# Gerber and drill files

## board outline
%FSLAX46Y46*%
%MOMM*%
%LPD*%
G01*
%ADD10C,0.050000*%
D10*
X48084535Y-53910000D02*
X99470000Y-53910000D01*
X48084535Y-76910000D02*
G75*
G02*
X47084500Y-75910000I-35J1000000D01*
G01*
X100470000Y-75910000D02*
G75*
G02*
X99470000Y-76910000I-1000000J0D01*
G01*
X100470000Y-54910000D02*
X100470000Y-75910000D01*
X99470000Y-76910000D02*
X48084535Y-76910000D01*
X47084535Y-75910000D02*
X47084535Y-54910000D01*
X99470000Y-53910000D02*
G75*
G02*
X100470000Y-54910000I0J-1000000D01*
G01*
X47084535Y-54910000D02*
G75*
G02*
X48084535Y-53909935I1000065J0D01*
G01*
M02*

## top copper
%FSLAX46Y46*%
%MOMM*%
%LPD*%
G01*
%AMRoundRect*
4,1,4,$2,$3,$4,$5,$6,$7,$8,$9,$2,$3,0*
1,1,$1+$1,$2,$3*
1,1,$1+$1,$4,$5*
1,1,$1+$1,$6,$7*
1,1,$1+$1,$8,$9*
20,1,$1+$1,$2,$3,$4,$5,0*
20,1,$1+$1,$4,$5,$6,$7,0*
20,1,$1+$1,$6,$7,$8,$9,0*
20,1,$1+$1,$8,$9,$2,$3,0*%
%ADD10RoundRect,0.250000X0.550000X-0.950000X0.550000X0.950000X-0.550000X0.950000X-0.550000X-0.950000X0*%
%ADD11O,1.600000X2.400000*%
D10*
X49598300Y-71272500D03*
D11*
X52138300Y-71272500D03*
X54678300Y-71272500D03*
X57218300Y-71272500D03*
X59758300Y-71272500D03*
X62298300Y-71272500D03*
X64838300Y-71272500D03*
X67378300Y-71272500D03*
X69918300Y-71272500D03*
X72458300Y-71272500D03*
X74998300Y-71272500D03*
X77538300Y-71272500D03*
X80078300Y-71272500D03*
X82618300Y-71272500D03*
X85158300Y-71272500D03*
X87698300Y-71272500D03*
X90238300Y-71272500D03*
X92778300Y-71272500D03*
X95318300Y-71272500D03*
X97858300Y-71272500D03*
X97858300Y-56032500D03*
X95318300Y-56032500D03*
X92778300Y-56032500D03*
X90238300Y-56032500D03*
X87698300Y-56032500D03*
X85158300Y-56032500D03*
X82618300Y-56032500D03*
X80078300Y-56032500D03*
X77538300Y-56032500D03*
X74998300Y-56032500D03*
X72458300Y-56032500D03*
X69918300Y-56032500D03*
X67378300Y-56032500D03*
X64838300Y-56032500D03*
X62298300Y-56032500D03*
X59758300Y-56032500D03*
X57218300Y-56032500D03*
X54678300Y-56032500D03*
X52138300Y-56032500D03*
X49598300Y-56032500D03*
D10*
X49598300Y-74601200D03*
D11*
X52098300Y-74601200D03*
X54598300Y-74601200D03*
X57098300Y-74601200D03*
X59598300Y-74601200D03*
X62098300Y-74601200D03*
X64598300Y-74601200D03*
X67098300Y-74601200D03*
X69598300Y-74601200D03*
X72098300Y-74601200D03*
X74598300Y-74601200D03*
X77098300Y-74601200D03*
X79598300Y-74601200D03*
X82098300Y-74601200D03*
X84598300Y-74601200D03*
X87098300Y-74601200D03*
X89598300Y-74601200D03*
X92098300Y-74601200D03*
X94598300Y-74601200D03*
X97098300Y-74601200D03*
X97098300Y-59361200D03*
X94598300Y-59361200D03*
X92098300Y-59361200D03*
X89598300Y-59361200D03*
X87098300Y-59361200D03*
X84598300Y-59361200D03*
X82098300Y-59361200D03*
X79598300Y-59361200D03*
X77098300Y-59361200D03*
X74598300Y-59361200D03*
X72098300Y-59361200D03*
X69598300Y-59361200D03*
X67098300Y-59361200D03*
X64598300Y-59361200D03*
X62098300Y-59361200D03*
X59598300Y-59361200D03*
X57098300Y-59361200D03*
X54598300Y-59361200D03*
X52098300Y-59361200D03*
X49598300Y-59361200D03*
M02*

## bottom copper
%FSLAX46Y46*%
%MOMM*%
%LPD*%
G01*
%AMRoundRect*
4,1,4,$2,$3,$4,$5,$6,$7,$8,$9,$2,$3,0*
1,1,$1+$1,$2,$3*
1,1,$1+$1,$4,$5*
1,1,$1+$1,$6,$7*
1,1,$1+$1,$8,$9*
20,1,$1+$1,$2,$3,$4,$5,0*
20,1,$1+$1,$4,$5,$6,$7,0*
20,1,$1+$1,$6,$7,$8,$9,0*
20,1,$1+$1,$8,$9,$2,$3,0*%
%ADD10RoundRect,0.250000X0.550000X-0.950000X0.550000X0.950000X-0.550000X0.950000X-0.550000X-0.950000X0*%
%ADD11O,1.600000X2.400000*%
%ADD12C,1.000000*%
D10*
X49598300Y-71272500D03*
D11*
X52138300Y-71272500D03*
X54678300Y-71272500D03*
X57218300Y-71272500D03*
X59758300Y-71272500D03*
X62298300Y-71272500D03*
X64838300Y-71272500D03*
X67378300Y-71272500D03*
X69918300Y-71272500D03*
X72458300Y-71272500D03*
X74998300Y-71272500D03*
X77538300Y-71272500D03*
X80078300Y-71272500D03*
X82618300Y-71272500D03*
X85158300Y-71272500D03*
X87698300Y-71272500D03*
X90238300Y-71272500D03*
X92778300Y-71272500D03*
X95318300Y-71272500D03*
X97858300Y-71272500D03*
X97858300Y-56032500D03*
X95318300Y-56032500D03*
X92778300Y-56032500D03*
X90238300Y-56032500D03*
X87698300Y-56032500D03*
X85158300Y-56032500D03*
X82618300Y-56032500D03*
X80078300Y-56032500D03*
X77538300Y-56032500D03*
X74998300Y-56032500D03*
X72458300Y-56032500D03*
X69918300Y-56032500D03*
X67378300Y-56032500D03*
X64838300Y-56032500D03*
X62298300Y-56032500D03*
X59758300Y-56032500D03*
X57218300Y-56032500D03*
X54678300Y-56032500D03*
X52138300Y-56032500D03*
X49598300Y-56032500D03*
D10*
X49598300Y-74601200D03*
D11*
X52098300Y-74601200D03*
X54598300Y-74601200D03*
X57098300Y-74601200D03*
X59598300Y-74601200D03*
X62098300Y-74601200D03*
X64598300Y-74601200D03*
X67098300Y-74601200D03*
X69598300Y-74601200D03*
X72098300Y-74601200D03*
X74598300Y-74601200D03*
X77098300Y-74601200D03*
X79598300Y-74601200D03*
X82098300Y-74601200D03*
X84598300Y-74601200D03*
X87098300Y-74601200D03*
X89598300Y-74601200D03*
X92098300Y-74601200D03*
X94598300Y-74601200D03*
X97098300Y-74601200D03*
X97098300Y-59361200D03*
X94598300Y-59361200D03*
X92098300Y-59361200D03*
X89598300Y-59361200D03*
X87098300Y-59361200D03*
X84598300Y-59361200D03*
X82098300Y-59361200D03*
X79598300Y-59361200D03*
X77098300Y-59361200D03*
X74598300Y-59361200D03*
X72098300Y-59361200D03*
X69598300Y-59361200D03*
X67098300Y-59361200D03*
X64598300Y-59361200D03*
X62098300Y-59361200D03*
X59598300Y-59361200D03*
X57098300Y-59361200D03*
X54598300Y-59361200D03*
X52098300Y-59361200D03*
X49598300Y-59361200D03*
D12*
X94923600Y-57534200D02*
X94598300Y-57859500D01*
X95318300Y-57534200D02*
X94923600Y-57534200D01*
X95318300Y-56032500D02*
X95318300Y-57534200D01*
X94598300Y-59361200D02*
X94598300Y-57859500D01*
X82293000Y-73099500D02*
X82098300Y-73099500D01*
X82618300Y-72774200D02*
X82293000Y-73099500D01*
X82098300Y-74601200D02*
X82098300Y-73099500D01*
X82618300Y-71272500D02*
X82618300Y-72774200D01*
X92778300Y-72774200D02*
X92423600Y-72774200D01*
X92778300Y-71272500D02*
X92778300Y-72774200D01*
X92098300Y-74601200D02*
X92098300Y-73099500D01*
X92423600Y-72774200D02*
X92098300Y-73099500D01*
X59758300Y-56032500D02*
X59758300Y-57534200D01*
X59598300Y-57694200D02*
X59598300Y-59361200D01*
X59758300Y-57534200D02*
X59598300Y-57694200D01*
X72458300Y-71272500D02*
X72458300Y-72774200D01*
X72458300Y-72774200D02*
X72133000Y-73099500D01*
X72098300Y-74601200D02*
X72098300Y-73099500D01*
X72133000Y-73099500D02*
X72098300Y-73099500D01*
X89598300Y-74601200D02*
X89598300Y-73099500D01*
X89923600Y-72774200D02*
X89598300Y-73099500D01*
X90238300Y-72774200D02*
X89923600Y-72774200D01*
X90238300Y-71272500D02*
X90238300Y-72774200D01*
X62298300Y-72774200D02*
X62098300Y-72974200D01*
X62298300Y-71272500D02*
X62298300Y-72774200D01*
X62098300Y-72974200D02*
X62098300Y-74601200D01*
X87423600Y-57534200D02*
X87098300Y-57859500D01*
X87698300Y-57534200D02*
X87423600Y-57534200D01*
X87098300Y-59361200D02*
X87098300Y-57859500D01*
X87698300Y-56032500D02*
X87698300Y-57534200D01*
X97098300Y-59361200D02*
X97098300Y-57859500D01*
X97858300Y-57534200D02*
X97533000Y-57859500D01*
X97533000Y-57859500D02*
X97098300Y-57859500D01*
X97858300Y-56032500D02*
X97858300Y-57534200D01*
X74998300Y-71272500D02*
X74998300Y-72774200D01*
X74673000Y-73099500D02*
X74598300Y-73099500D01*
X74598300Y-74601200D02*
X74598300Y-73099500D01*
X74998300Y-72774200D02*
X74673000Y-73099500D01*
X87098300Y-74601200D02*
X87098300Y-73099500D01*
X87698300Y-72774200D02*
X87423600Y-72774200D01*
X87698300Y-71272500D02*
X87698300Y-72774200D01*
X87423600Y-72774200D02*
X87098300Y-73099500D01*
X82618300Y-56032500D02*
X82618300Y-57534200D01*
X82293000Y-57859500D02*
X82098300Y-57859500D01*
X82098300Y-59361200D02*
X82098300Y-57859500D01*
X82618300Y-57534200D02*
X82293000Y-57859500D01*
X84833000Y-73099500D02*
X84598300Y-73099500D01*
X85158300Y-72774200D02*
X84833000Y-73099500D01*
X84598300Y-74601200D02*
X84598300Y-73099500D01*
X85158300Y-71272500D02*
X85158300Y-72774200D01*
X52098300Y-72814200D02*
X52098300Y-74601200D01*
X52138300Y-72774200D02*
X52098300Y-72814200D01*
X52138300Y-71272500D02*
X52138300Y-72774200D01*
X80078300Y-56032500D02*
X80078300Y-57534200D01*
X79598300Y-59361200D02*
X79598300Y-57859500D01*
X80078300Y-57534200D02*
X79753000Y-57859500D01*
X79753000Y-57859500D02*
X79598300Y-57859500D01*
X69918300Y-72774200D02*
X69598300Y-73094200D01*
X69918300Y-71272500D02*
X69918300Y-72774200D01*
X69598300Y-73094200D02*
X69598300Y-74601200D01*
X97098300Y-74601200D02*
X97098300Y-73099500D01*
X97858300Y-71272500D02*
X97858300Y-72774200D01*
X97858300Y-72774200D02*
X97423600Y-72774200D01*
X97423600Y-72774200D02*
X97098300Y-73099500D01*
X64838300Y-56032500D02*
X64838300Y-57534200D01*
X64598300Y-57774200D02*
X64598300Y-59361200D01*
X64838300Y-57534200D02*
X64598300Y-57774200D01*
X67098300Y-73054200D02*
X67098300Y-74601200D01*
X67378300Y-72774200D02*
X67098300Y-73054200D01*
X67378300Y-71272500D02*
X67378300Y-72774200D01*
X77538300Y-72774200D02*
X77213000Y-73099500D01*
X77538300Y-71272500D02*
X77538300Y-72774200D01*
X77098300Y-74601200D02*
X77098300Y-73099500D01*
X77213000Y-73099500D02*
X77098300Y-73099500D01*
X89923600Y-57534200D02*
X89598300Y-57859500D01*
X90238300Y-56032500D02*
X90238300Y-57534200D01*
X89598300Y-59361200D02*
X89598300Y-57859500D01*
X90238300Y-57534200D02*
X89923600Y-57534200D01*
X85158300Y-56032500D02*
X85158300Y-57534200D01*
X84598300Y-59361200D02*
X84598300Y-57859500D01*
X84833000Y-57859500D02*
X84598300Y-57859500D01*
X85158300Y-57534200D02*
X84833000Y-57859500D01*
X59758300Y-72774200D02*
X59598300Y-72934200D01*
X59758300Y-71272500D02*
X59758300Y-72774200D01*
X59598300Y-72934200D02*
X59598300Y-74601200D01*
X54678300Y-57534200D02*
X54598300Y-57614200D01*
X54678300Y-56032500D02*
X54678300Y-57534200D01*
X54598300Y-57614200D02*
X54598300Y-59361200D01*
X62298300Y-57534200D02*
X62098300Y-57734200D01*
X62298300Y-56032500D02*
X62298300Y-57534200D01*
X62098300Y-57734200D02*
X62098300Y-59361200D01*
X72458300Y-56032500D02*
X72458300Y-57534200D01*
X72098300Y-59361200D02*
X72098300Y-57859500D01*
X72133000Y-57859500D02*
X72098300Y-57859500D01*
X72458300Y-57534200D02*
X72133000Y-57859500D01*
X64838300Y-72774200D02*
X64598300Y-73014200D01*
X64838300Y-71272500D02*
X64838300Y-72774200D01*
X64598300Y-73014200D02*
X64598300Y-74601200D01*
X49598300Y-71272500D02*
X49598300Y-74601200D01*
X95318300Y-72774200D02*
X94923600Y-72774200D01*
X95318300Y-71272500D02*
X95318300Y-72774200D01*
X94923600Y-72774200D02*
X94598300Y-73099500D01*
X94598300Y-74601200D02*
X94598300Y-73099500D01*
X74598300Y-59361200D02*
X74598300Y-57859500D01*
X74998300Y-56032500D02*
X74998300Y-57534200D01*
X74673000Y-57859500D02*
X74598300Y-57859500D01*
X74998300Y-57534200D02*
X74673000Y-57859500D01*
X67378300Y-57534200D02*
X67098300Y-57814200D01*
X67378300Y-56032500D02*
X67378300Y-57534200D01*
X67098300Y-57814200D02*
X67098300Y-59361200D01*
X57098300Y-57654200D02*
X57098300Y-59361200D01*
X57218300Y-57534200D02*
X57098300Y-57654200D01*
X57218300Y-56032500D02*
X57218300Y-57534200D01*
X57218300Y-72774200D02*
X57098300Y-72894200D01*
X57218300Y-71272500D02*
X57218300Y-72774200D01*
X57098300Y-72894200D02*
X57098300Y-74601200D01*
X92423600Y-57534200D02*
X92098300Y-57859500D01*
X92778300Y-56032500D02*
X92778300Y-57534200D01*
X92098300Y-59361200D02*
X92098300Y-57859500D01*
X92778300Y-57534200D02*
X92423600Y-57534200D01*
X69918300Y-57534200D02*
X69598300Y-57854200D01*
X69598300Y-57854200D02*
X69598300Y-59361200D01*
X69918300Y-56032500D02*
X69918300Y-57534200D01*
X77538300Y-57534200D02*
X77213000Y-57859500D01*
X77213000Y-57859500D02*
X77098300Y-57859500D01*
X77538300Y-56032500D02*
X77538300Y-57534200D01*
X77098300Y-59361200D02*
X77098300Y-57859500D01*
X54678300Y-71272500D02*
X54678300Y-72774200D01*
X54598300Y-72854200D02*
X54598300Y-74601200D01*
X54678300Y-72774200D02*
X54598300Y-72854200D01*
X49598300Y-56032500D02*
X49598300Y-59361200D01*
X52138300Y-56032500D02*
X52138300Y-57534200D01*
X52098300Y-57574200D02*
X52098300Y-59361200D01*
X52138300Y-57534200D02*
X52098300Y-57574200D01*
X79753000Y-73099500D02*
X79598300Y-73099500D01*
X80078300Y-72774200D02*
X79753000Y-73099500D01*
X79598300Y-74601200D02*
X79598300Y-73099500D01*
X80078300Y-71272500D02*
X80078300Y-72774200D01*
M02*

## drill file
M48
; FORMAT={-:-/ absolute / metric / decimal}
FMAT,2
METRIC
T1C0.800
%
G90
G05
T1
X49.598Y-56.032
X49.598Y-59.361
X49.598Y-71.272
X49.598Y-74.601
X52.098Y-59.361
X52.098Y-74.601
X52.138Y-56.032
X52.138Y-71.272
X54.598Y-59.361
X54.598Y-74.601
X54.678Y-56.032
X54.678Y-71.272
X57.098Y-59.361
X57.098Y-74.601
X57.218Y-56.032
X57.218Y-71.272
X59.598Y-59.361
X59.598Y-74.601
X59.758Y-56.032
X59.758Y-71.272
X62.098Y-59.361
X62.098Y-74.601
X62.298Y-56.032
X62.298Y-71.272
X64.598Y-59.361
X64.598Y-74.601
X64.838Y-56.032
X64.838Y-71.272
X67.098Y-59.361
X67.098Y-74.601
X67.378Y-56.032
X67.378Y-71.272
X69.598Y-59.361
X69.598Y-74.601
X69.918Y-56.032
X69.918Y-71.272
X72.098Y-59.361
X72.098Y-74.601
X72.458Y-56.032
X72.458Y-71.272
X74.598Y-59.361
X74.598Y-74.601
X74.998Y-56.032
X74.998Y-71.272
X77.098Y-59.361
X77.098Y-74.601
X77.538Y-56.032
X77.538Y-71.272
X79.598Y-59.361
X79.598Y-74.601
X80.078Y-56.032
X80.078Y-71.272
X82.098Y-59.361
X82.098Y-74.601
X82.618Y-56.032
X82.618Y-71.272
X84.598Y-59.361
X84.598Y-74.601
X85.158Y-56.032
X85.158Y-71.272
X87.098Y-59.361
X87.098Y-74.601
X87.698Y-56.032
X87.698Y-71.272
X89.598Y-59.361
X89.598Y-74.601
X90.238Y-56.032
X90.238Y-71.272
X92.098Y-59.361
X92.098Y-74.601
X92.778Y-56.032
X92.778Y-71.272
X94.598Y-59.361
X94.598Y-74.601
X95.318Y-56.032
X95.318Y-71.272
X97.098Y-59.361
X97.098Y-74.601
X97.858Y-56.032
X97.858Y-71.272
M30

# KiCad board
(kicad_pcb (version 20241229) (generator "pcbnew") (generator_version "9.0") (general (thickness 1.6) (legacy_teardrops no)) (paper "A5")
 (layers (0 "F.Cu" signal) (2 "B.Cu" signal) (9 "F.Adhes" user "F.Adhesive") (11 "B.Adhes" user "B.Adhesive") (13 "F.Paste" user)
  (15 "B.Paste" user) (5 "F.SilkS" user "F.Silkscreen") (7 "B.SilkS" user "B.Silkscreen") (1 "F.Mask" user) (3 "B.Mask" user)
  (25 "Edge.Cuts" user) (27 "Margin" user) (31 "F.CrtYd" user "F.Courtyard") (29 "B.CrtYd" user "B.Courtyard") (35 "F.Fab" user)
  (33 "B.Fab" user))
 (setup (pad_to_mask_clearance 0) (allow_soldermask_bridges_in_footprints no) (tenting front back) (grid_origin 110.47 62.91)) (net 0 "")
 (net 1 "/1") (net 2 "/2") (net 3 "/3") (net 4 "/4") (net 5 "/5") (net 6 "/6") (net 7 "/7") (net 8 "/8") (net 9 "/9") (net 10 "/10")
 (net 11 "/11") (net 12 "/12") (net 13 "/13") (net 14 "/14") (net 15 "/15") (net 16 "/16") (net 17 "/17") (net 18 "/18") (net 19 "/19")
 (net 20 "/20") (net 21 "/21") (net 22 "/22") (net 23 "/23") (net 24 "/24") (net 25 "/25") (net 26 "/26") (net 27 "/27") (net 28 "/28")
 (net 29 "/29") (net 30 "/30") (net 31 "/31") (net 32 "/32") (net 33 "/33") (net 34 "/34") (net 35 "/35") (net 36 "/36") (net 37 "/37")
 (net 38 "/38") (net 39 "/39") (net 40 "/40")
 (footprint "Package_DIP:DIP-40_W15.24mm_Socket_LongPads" (layer "F.Cu") (at 49.5983 71.2725 90)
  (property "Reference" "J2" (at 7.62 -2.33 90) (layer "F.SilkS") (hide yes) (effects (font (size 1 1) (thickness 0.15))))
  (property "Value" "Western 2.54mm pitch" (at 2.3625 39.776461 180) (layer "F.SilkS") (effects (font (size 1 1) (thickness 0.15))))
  (pad "1" thru_hole roundrect (at 0 0 90) (size 2.4 1.6) (drill 0.8) (layers "*.Cu" "*.Mask") (remove_unused_layers no)
   (roundrect_rratio 0.15625) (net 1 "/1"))
  (pad "2" thru_hole oval (at 0 2.54 90) (size 2.4 1.6) (drill 0.8) (layers "*.Cu" "*.Mask") (remove_unused_layers no) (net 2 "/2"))
  (pad "3" thru_hole oval (at 0 5.08 90) (size 2.4 1.6) (drill 0.8) (layers "*.Cu" "*.Mask") (remove_unused_layers no) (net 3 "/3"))
  (pad "4" thru_hole oval (at 0 7.62 90) (size 2.4 1.6) (drill 0.8) (layers "*.Cu" "*.Mask") (remove_unused_layers no) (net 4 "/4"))
  (pad "5" thru_hole oval (at 0 10.16 90) (size 2.4 1.6) (drill 0.8) (layers "*.Cu" "*.Mask") (remove_unused_layers no) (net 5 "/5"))
  (pad "6" thru_hole oval (at 0 12.7 90) (size 2.4 1.6) (drill 0.8) (layers "*.Cu" "*.Mask") (remove_unused_layers no) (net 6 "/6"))
  (pad "7" thru_hole oval (at 0 15.24 90) (size 2.4 1.6) (drill 0.8) (layers "*.Cu" "*.Mask") (remove_unused_layers no) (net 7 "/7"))
  (pad "8" thru_hole oval (at 0 17.78 90) (size 2.4 1.6) (drill 0.8) (layers "*.Cu" "*.Mask") (remove_unused_layers no) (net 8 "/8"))
  (pad "9" thru_hole oval (at 0 20.32 90) (size 2.4 1.6) (drill 0.8) (layers "*.Cu" "*.Mask") (remove_unused_layers no) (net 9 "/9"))
  (pad "10" thru_hole oval (at 0 22.86 90) (size 2.4 1.6) (drill 0.8) (layers "*.Cu" "*.Mask") (remove_unused_layers no) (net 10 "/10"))
  (pad "11" thru_hole oval (at 0 25.4 90) (size 2.4 1.6) (drill 0.8) (layers "*.Cu" "*.Mask") (remove_unused_layers no) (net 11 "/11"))
  (pad "12" thru_hole oval (at 0 27.94 90) (size 2.4 1.6) (drill 0.8) (layers "*.Cu" "*.Mask") (remove_unused_layers no) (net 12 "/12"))
  (pad "13" thru_hole oval (at 0 30.48 90) (size 2.4 1.6) (drill 0.8) (layers "*.Cu" "*.Mask") (remove_unused_layers no) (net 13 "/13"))
  (pad "14" thru_hole oval (at 0 33.02 90) (size 2.4 1.6) (drill 0.8) (layers "*.Cu" "*.Mask") (remove_unused_layers no) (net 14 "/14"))
  (pad "15" thru_hole oval (at 0 35.56 90) (size 2.4 1.6) (drill 0.8) (layers "*.Cu" "*.Mask") (remove_unused_layers no) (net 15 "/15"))
  (pad "16" thru_hole oval (at 0 38.1 90) (size 2.4 1.6) (drill 0.8) (layers "*.Cu" "*.Mask") (remove_unused_layers no) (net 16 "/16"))
  (pad "17" thru_hole oval (at 0 40.64 90) (size 2.4 1.6) (drill 0.8) (layers "*.Cu" "*.Mask") (remove_unused_layers no) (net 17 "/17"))
  (pad "18" thru_hole oval (at 0 43.18 90) (size 2.4 1.6) (drill 0.8) (layers "*.Cu" "*.Mask") (remove_unused_layers no) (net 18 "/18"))
  (pad "19" thru_hole oval (at 0 45.72 90) (size 2.4 1.6) (drill 0.8) (layers "*.Cu" "*.Mask") (remove_unused_layers no) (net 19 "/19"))
  (pad "20" thru_hole oval (at 0 48.26 90) (size 2.4 1.6) (drill 0.8) (layers "*.Cu" "*.Mask") (remove_unused_layers no) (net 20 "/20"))
  (pad "21" thru_hole oval (at 15.24 48.26 90) (size 2.4 1.6) (drill 0.8) (layers "*.Cu" "*.Mask") (remove_unused_layers no) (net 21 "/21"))
  (pad "22" thru_hole oval (at 15.24 45.72 90) (size 2.4 1.6) (drill 0.8) (layers "*.Cu" "*.Mask") (remove_unused_layers no) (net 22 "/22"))
  (pad "23" thru_hole oval (at 15.24 43.18 90) (size 2.4 1.6) (drill 0.8) (layers "*.Cu" "*.Mask") (remove_unused_layers no) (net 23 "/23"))
  (pad "24" thru_hole oval (at 15.24 40.64 90) (size 2.4 1.6) (drill 0.8) (layers "*.Cu" "*.Mask") (remove_unused_layers no) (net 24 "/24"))
  (pad "25" thru_hole oval (at 15.24 38.1 90) (size 2.4 1.6) (drill 0.8) (layers "*.Cu" "*.Mask") (remove_unused_layers no) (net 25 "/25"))
  (pad "26" thru_hole oval (at 15.24 35.56 90) (size 2.4 1.6) (drill 0.8) (layers "*.Cu" "*.Mask") (remove_unused_layers no) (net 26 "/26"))
  (pad "27" thru_hole oval (at 15.24 33.02 90) (size 2.4 1.6) (drill 0.8) (layers "*.Cu" "*.Mask") (remove_unused_layers no) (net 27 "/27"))
  (pad "28" thru_hole oval (at 15.24 30.48 90) (size 2.4 1.6) (drill 0.8) (layers "*.Cu" "*.Mask") (remove_unused_layers no) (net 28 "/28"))
  (pad "29" thru_hole oval (at 15.24 27.94 90) (size 2.4 1.6) (drill 0.8) (layers "*.Cu" "*.Mask") (remove_unused_layers no) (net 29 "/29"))
  (pad "30" thru_hole oval (at 15.24 25.4 90) (size 2.4 1.6) (drill 0.8) (layers "*.Cu" "*.Mask") (remove_unused_layers no) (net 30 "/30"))
  (pad "31" thru_hole oval (at 15.24 22.86 90) (size 2.4 1.6) (drill 0.8) (layers "*.Cu" "*.Mask") (remove_unused_layers no) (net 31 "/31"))
  (pad "32" thru_hole oval (at 15.24 20.32 90) (size 2.4 1.6) (drill 0.8) (layers "*.Cu" "*.Mask") (remove_unused_layers no) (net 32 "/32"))
  (pad "33" thru_hole oval (at 15.24 17.78 90) (size 2.4 1.6) (drill 0.8) (layers "*.Cu" "*.Mask") (remove_unused_layers no) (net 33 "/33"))
  (pad "34" thru_hole oval (at 15.24 15.24 90) (size 2.4 1.6) (drill 0.8) (layers "*.Cu" "*.Mask") (remove_unused_layers no) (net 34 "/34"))
  (pad "35" thru_hole oval (at 15.24 12.7 90) (size 2.4 1.6) (drill 0.8) (layers "*.Cu" "*.Mask") (remove_unused_layers no) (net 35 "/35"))
  (pad "36" thru_hole oval (at 15.24 10.16 90) (size 2.4 1.6) (drill 0.8) (layers "*.Cu" "*.Mask") (remove_unused_layers no) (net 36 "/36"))
  (pad "37" thru_hole oval (at 15.24 7.62 90) (size 2.4 1.6) (drill 0.8) (layers "*.Cu" "*.Mask") (remove_unused_layers no) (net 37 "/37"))
  (pad "38" thru_hole oval (at 15.24 5.08 90) (size 2.4 1.6) (drill 0.8) (layers "*.Cu" "*.Mask") (remove_unused_layers no) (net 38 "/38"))
  (pad "39" thru_hole oval (at 15.24 2.54 90) (size 2.4 1.6) (drill 0.8) (layers "*.Cu" "*.Mask") (remove_unused_layers no) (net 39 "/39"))
  (pad "40" thru_hole oval (at 15.24 0 90) (size 2.4 1.6) (drill 0.8) (layers "*.Cu" "*.Mask") (remove_unused_layers no) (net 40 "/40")))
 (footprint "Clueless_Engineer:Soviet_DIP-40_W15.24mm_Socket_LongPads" (layer "F.Cu") (at 49.5983 74.6012 90)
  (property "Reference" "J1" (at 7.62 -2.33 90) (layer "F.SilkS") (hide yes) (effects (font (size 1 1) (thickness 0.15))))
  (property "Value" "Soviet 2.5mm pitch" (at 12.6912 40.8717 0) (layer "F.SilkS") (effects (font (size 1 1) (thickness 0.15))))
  (pad "1" thru_hole roundrect (at 0 0 90) (size 2.4 1.6) (drill 0.8) (layers "*.Cu" "*.Mask") (remove_unused_layers no)
   (roundrect_rratio 0.15625) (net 1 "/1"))
  (pad "2" thru_hole oval (at 0 2.5 90) (size 2.4 1.6) (drill 0.8) (layers "*.Cu" "*.Mask") (remove_unused_layers no) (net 2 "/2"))
  (pad "3" thru_hole oval (at 0 5 90) (size 2.4 1.6) (drill 0.8) (layers "*.Cu" "*.Mask") (remove_unused_layers no) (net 3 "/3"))
  (pad "4" thru_hole oval (at 0 7.5 90) (size 2.4 1.6) (drill 0.8) (layers "*.Cu" "*.Mask") (remove_unused_layers no) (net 4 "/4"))
  (pad "5" thru_hole oval (at 0 10 90) (size 2.4 1.6) (drill 0.8) (layers "*.Cu" "*.Mask") (remove_unused_layers no) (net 5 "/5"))
  (pad "6" thru_hole oval (at 0 12.5 90) (size 2.4 1.6) (drill 0.8) (layers "*.Cu" "*.Mask") (remove_unused_layers no) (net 6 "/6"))
  (pad "7" thru_hole oval (at 0 15 90) (size 2.4 1.6) (drill 0.8) (layers "*.Cu" "*.Mask") (remove_unused_layers no) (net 7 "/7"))
  (pad "8" thru_hole oval (at 0 17.5 90) (size 2.4 1.6) (drill 0.8) (layers "*.Cu" "*.Mask") (remove_unused_layers no) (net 8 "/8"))
  (pad "9" thru_hole oval (at 0 20 90) (size 2.4 1.6) (drill 0.8) (layers "*.Cu" "*.Mask") (remove_unused_layers no) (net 9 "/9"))
  (pad "10" thru_hole oval (at 0 22.5 90) (size 2.4 1.6) (drill 0.8) (layers "*.Cu" "*.Mask") (remove_unused_layers no) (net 10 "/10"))
  (pad "11" thru_hole oval (at 0 25 90) (size 2.4 1.6) (drill 0.8) (layers "*.Cu" "*.Mask") (remove_unused_layers no) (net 11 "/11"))
  (pad "12" thru_hole oval (at 0 27.5 90) (size 2.4 1.6) (drill 0.8) (layers "*.Cu" "*.Mask") (remove_unused_layers no) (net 12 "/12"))
  (pad "13" thru_hole oval (at 0 30 90) (size 2.4 1.6) (drill 0.8) (layers "*.Cu" "*.Mask") (remove_unused_layers no) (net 13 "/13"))
  (pad "14" thru_hole oval (at 0 32.5 90) (size 2.4 1.6) (drill 0.8) (layers "*.Cu" "*.Mask") (remove_unused_layers no) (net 14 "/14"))
  (pad "15" thru_hole oval (at 0 35 90) (size 2.4 1.6) (drill 0.8) (layers "*.Cu" "*.Mask") (remove_unused_layers no) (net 15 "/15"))
  (pad "16" thru_hole oval (at 0 37.5 90) (size 2.4 1.6) (drill 0.8) (layers "*.Cu" "*.Mask") (remove_unused_layers no) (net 16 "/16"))
  (pad "17" thru_hole oval (at 0 40 90) (size 2.4 1.6) (drill 0.8) (layers "*.Cu" "*.Mask") (remove_unused_layers no) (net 17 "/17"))
  (pad "18" thru_hole oval (at 0 42.5 90) (size 2.4 1.6) (drill 0.8) (layers "*.Cu" "*.Mask") (remove_unused_layers no) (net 18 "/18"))
  (pad "19" thru_hole oval (at 0 45 90) (size 2.4 1.6) (drill 0.8) (layers "*.Cu" "*.Mask") (remove_unused_layers no) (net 19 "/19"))
  (pad "20" thru_hole oval (at 0 47.5 90) (size 2.4 1.6) (drill 0.8) (layers "*.Cu" "*.Mask") (remove_unused_layers no) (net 20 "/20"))
  (pad "21" thru_hole oval (at 15.24 47.5 90) (size 2.4 1.6) (drill 0.8) (layers "*.Cu" "*.Mask") (remove_unused_layers no) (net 21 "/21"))
  (pad "22" thru_hole oval (at 15.24 45 90) (size 2.4 1.6) (drill 0.8) (layers "*.Cu" "*.Mask") (remove_unused_layers no) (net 22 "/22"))
  (pad "23" thru_hole oval (at 15.24 42.5 90) (size 2.4 1.6) (drill 0.8) (layers "*.Cu" "*.Mask") (remove_unused_layers no) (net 23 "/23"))
  (pad "24" thru_hole oval (at 15.24 40 90) (size 2.4 1.6) (drill 0.8) (layers "*.Cu" "*.Mask") (remove_unused_layers no) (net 24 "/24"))
  (pad "25" thru_hole oval (at 15.24 37.5 90) (size 2.4 1.6) (drill 0.8) (layers "*.Cu" "*.Mask") (remove_unused_layers no) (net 25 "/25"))
  (pad "26" thru_hole oval (at 15.24 35 90) (size 2.4 1.6) (drill 0.8) (layers "*.Cu" "*.Mask") (remove_unused_layers no) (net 26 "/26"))
  (pad "27" thru_hole oval (at 15.24 32.5 90) (size 2.4 1.6) (drill 0.8) (layers "*.Cu" "*.Mask") (remove_unused_layers no) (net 27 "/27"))
  (pad "28" thru_hole oval (at 15.24 30 90) (size 2.4 1.6) (drill 0.8) (layers "*.Cu" "*.Mask") (remove_unused_layers no) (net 28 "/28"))
  (pad "29" thru_hole oval (at 15.24 27.5 90) (size 2.4 1.6) (drill 0.8) (layers "*.Cu" "*.Mask") (remove_unused_layers no) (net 29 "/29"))
  (pad "30" thru_hole oval (at 15.24 25 90) (size 2.4 1.6) (drill 0.8) (layers "*.Cu" "*.Mask") (remove_unused_layers no) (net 30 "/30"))
  (pad "31" thru_hole oval (at 15.24 22.5 90) (size 2.4 1.6) (drill 0.8) (layers "*.Cu" "*.Mask") (remove_unused_layers no) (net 31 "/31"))
  (pad "32" thru_hole oval (at 15.24 20 90) (size 2.4 1.6) (drill 0.8) (layers "*.Cu" "*.Mask") (remove_unused_layers no) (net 32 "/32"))
  (pad "33" thru_hole oval (at 15.24 17.5 90) (size 2.4 1.6) (drill 0.8) (layers "*.Cu" "*.Mask") (remove_unused_layers no) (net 33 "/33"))
  (pad "34" thru_hole oval (at 15.24 15 90) (size 2.4 1.6) (drill 0.8) (layers "*.Cu" "*.Mask") (remove_unused_layers no) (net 34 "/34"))
  (pad "35" thru_hole oval (at 15.24 12.5 90) (size 2.4 1.6) (drill 0.8) (layers "*.Cu" "*.Mask") (remove_unused_layers no) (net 35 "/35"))
  (pad "36" thru_hole oval (at 15.24 10 90) (size 2.4 1.6) (drill 0.8) (layers "*.Cu" "*.Mask") (remove_unused_layers no) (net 36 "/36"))
  (pad "37" thru_hole oval (at 15.24 7.5 90) (size 2.4 1.6) (drill 0.8) (layers "*.Cu" "*.Mask") (remove_unused_layers no) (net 37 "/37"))
  (pad "38" thru_hole oval (at 15.24 5 90) (size 2.4 1.6) (drill 0.8) (layers "*.Cu" "*.Mask") (remove_unused_layers no) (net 38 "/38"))
  (pad "39" thru_hole oval (at 15.24 2.5 90) (size 2.4 1.6) (drill 0.8) (layers "*.Cu" "*.Mask") (remove_unused_layers no) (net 39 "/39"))
  (pad "40" thru_hole oval (at 15.24 0 90) (size 2.4 1.6) (drill 0.8) (layers "*.Cu" "*.Mask") (remove_unused_layers no) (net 40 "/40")))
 (gr_line (start 48.084535 53.91) (end 99.47 53.91) (stroke (width 0.05) (type default)) (layer "Edge.Cuts"))
 (gr_arc (start 48.084535 76.91) (mid 47.377428 76.617107) (end 47.084535 75.91) (stroke (width 0.05) (type default)) (layer "Edge.Cuts"))
 (gr_arc (start 100.47 75.91) (mid 100.177107 76.617107) (end 99.47 76.91) (stroke (width 0.05) (type default)) (layer "Edge.Cuts"))
 (gr_line (start 100.47 54.91) (end 100.47 75.91) (stroke (width 0.05) (type default)) (layer "Edge.Cuts"))
 (gr_line (start 99.47 76.91) (end 48.084535 76.91) (stroke (width 0.05) (type default)) (layer "Edge.Cuts"))
 (gr_line (start 47.084535 75.91) (end 47.084535 54.91) (stroke (width 0.05) (type default)) (layer "Edge.Cuts"))
 (gr_arc (start 99.47 53.91) (mid 100.177107 54.202893) (end 100.47 54.91) (stroke (width 0.05) (type default)) (layer "Edge.Cuts"))
 (gr_arc (start 47.084535 54.91) (mid 47.37743 54.202906) (end 48.084535 53.91) (stroke (width 0.05) (type default)) (layer "Edge.Cuts"))
 (segment (start 94.9236 57.5342) (end 94.5983 57.8595) (width 1) (layer "B.Cu") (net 22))
 (segment (start 95.3183 57.5342) (end 94.9236 57.5342) (width 1) (layer "B.Cu") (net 22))
 (segment (start 95.3183 56.0325) (end 95.3183 57.5342) (width 1) (layer "B.Cu") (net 22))
 (segment (start 94.5983 59.3612) (end 94.5983 57.8595) (width 1) (layer "B.Cu") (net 22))
 (segment (start 82.293 73.0995) (end 82.0983 73.0995) (width 1) (layer "B.Cu") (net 14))
 (segment (start 82.6183 72.7742) (end 82.293 73.0995) (width 1) (layer "B.Cu") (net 14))
 (segment (start 82.0983 74.6012) (end 82.0983 73.0995) (width 1) (layer "B.Cu") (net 14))
 (segment (start 82.6183 71.2725) (end 82.6183 72.7742) (width 1) (layer "B.Cu") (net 14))
 (segment (start 92.7783 72.7742) (end 92.4236 72.7742) (width 1) (layer "B.Cu") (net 18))
 (segment (start 92.7783 71.2725) (end 92.7783 72.7742) (width 1) (layer "B.Cu") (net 18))
 (segment (start 92.0983 74.6012) (end 92.0983 73.0995) (width 1) (layer "B.Cu") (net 18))
 (segment (start 92.4236 72.7742) (end 92.0983 73.0995) (width 1) (layer "B.Cu") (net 18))
 (segment (start 59.7583 56.0325) (end 59.7583 57.5342) (width 1) (layer "B.Cu") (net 36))
 (segment (start 59.5983 57.6942) (end 59.5983 59.3612) (width 1) (layer "B.Cu") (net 36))
 (segment (start 59.7583 57.5342) (end 59.5983 57.6942) (width 1) (layer "B.Cu") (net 36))
 (segment (start 72.4583 71.2725) (end 72.4583 72.7742) (width 1) (layer "B.Cu") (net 10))
 (segment (start 72.4583 72.7742) (end 72.133 73.0995) (width 1) (layer "B.Cu") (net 10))
 (segment (start 72.0983 74.6012) (end 72.0983 73.0995) (width 1) (layer "B.Cu") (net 10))
 (segment (start 72.133 73.0995) (end 72.0983 73.0995) (width 1) (layer "B.Cu") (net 10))
 (segment (start 89.5983 74.6012) (end 89.5983 73.0995) (width 1) (layer "B.Cu") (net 17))
 (segment (start 89.9236 72.7742) (end 89.5983 73.0995) (width 1) (layer "B.Cu") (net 17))
 (segment (start 90.2383 72.7742) (end 89.9236 72.7742) (width 1) (layer "B.Cu") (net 17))
 (segment (start 90.2383 71.2725) (end 90.2383 72.7742) (width 1) (layer "B.Cu") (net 17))
 (segment (start 62.2983 72.7742) (end 62.0983 72.9742) (width 1) (layer "B.Cu") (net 6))
 (segment (start 62.2983 71.2725) (end 62.2983 72.7742) (width 1) (layer "B.Cu") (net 6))
 (segment (start 62.0983 72.9742) (end 62.0983 74.6012) (width 1) (layer "B.Cu") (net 6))
 (segment (start 87.4236 57.5342) (end 87.0983 57.8595) (width 1) (layer "B.Cu") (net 25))
 (segment (start 87.6983 57.5342) (end 87.4236 57.5342) (width 1) (layer "B.Cu") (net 25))
 (segment (start 87.0983 59.3612) (end 87.0983 57.8595) (width 1) (layer "B.Cu") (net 25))
 (segment (start 87.6983 56.0325) (end 87.6983 57.5342) (width 1) (layer "B.Cu") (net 25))
 (segment (start 97.0983 59.3612) (end 97.0983 57.8595) (width 1) (layer "B.Cu") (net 21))
 (segment (start 97.8583 57.5342) (end 97.533 57.8595) (width 1) (layer "B.Cu") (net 21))
 (segment (start 97.533 57.8595) (end 97.0983 57.8595) (width 1) (layer "B.Cu") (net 21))
 (segment (start 97.8583 56.0325) (end 97.8583 57.5342) (width 1) (layer "B.Cu") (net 21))
 (segment (start 74.9983 71.2725) (end 74.9983 72.7742) (width 1) (layer "B.Cu") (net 11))
 (segment (start 74.673 73.0995) (end 74.5983 73.0995) (width 1) (layer "B.Cu") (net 11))
 (segment (start 74.5983 74.6012) (end 74.5983 73.0995) (width 1) (layer "B.Cu") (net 11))
 (segment (start 74.9983 72.7742) (end 74.673 73.0995) (width 1) (layer "B.Cu") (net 11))
 (segment (start 87.0983 74.6012) (end 87.0983 73.0995) (width 1) (layer "B.Cu") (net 16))
 (segment (start 87.6983 72.7742) (end 87.4236 72.7742) (width 1) (layer "B.Cu") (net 16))
 (segment (start 87.6983 71.2725) (end 87.6983 72.7742) (width 1) (layer "B.Cu") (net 16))
 (segment (start 87.4236 72.7742) (end 87.0983 73.0995) (width 1) (layer "B.Cu") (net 16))
 (segment (start 82.6183 56.0325) (end 82.6183 57.5342) (width 1) (layer "B.Cu") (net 27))
 (segment (start 82.293 57.8595) (end 82.0983 57.8595) (width 1) (layer "B.Cu") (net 27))
 (segment (start 82.0983 59.3612) (end 82.0983 57.8595) (width 1) (layer "B.Cu") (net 27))
 (segment (start 82.6183 57.5342) (end 82.293 57.8595) (width 1) (layer "B.Cu") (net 27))
 (segment (start 84.833 73.0995) (end 84.5983 73.0995) (width 1) (layer "B.Cu") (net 15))
 (segment (start 85.1583 72.7742) (end 84.833 73.0995) (width 1) (layer "B.Cu") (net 15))
 (segment (start 84.5983 74.6012) (end 84.5983 73.0995) (width 1) (layer "B.Cu") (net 15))
 (segment (start 85.1583 71.2725) (end 85.1583 72.7742) (width 1) (layer "B.Cu") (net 15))
 (segment (start 52.0983 72.8142) (end 52.0983 74.6012) (width 1) (layer "B.Cu") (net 2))
 (segment (start 52.1383 72.7742) (end 52.0983 72.8142) (width 1) (layer "B.Cu") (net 2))
 (segment (start 52.1383 71.2725) (end 52.1383 72.7742) (width 1) (layer "B.Cu") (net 2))
 (segment (start 80.0783 56.0325) (end 80.0783 57.5342) (width 1) (layer "B.Cu") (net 28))
 (segment (start 79.5983 59.3612) (end 79.5983 57.8595) (width 1) (layer "B.Cu") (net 28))
 (segment (start 80.0783 57.5342) (end 79.753 57.8595) (width 1) (layer "B.Cu") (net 28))
 (segment (start 79.753 57.8595) (end 79.5983 57.8595) (width 1) (layer "B.Cu") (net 28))
 (segment (start 69.9183 72.7742) (end 69.5983 73.0942) (width 1) (layer "B.Cu") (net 9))
 (segment (start 69.9183 71.2725) (end 69.9183 72.7742) (width 1) (layer "B.Cu") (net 9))
 (segment (start 69.5983 73.0942) (end 69.5983 74.6012) (width 1) (layer "B.Cu") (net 9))
 (segment (start 97.0983 74.6012) (end 97.0983 73.0995) (width 1) (layer "B.Cu") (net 20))
 (segment (start 97.8583 71.2725) (end 97.8583 72.7742) (width 1) (layer "B.Cu") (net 20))
 (segment (start 97.8583 72.7742) (end 97.4236 72.7742) (width 1) (layer "B.Cu") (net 20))
 (segment (start 97.4236 72.7742) (end 97.0983 73.0995) (width 1) (layer "B.Cu") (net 20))
 (segment (start 64.8383 56.0325) (end 64.8383 57.5342) (width 1) (layer "B.Cu") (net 34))
 (segment (start 64.5983 57.7742) (end 64.5983 59.3612) (width 1) (layer "B.Cu") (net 34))
 (segment (start 64.8383 57.5342) (end 64.5983 57.7742) (width 1) (layer "B.Cu") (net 34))
 (segment (start 67.0983 73.0542) (end 67.0983 74.6012) (width 1) (layer "B.Cu") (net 8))
 (segment (start 67.3783 72.7742) (end 67.0983 73.0542) (width 1) (layer "B.Cu") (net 8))
 (segment (start 67.3783 71.2725) (end 67.3783 72.7742) (width 1) (layer "B.Cu") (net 8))
 (segment (start 77.5383 72.7742) (end 77.213 73.0995) (width 1) (layer "B.Cu") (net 12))
 (segment (start 77.5383 71.2725) (end 77.5383 72.7742) (width 1) (layer "B.Cu") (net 12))
 (segment (start 77.0983 74.6012) (end 77.0983 73.0995) (width 1) (layer "B.Cu") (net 12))
 (segment (start 77.213 73.0995) (end 77.0983 73.0995) (width 1) (layer "B.Cu") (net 12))
 (segment (start 89.9236 57.5342) (end 89.5983 57.8595) (width 1) (layer "B.Cu") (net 24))
 (segment (start 90.2383 56.0325) (end 90.2383 57.5342) (width 1) (layer "B.Cu") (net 24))
 (segment (start 89.5983 59.3612) (end 89.5983 57.8595) (width 1) (layer "B.Cu") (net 24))
 (segment (start 90.2383 57.5342) (end 89.9236 57.5342) (width 1) (layer "B.Cu") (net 24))
 (segment (start 85.1583 56.0325) (end 85.1583 57.5342) (width 1) (layer "B.Cu") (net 26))
 (segment (start 84.5983 59.3612) (end 84.5983 57.8595) (width 1) (layer "B.Cu") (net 26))
 (segment (start 84.833 57.8595) (end 84.5983 57.8595) (width 1) (layer "B.Cu") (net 26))
 (segment (start 85.1583 57.5342) (end 84.833 57.8595) (width 1) (layer "B.Cu") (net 26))
 (segment (start 59.7583 72.7742) (end 59.5983 72.9342) (width 1) (layer "B.Cu") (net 5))
 (segment (start 59.7583 71.2725) (end 59.7583 72.7742) (width 1) (layer "B.Cu") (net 5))
 (segment (start 59.5983 72.9342) (end 59.5983 74.6012) (width 1) (layer "B.Cu") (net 5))
 (segment (start 54.6783 57.5342) (end 54.5983 57.6142) (width 1) (layer "B.Cu") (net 38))
 (segment (start 54.6783 56.0325) (end 54.6783 57.5342) (width 1) (layer "B.Cu") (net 38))
 (segment (start 54.5983 57.6142) (end 54.5983 59.3612) (width 1) (layer "B.Cu") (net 38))
 (segment (start 62.2983 57.5342) (end 62.0983 57.7342) (width 1) (layer "B.Cu") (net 35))
 (segment (start 62.2983 56.0325) (end 62.2983 57.5342) (width 1) (layer "B.Cu") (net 35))
 (segment (start 62.0983 57.7342) (end 62.0983 59.3612) (width 1) (layer "B.Cu") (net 35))
 (segment (start 72.4583 56.0325) (end 72.4583 57.5342) (width 1) (layer "B.Cu") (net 31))
 (segment (start 72.0983 59.3612) (end 72.0983 57.8595) (width 1) (layer "B.Cu") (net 31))
 (segment (start 72.133 57.8595) (end 72.0983 57.8595) (width 1) (layer "B.Cu") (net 31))
 (segment (start 72.4583 57.5342) (end 72.133 57.8595) (width 1) (layer "B.Cu") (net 31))
 (segment (start 64.8383 72.7742) (end 64.5983 73.0142) (width 1) (layer "B.Cu") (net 7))
 (segment (start 64.8383 71.2725) (end 64.8383 72.7742) (width 1) (layer "B.Cu") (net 7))
 (segment (start 64.5983 73.0142) (end 64.5983 74.6012) (width 1) (layer "B.Cu") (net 7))
 (segment (start 49.5983 71.2725) (end 49.5983 74.6012) (width 1) (layer "B.Cu") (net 1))
 (segment (start 95.3183 72.7742) (end 94.9236 72.7742) (width 1) (layer "B.Cu") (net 19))
 (segment (start 95.3183 71.2725) (end 95.3183 72.7742) (width 1) (layer "B.Cu") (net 19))
 (segment (start 94.9236 72.7742) (end 94.5983 73.0995) (width 1) (layer "B.Cu") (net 19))
 (segment (start 94.5983 74.6012) (end 94.5983 73.0995) (width 1) (layer "B.Cu") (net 19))
 (segment (start 74.5983 59.3612) (end 74.5983 57.8595) (width 1) (layer "B.Cu") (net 30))
 (segment (start 74.9983 56.0325) (end 74.9983 57.5342) (width 1) (layer "B.Cu") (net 30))
 (segment (start 74.673 57.8595) (end 74.5983 57.8595) (width 1) (layer "B.Cu") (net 30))
 (segment (start 74.9983 57.5342) (end 74.673 57.8595) (width 1) (layer "B.Cu") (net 30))
 (segment (start 67.3783 57.5342) (end 67.0983 57.8142) (width 1) (layer "B.Cu") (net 33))
 (segment (start 67.3783 56.0325) (end 67.3783 57.5342) (width 1) (layer "B.Cu") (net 33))
 (segment (start 67.0983 57.8142) (end 67.0983 59.3612) (width 1) (layer "B.Cu") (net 33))
 (segment (start 57.0983 57.6542) (end 57.0983 59.3612) (width 1) (layer "B.Cu") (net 37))
 (segment (start 57.2183 57.5342) (end 57.0983 57.6542) (width 1) (layer "B.Cu") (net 37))
 (segment (start 57.2183 56.0325) (end 57.2183 57.5342) (width 1) (layer "B.Cu") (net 37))
 (segment (start 57.2183 72.7742) (end 57.0983 72.8942) (width 1) (layer "B.Cu") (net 4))
 (segment (start 57.2183 71.2725) (end 57.2183 72.7742) (width 1) (layer "B.Cu") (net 4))
 (segment (start 57.0983 72.8942) (end 57.0983 74.6012) (width 1) (layer "B.Cu") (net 4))
 (segment (start 92.4236 57.5342) (end 92.0983 57.8595) (width 1) (layer "B.Cu") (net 23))
 (segment (start 92.7783 56.0325) (end 92.7783 57.5342) (width 1) (layer "B.Cu") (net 23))
 (segment (start 92.0983 59.3612) (end 92.0983 57.8595) (width 1) (layer "B.Cu") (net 23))
 (segment (start 92.7783 57.5342) (end 92.4236 57.5342) (width 1) (layer "B.Cu") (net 23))
 (segment (start 69.9183 57.5342) (end 69.5983 57.8542) (width 1) (layer "B.Cu") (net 32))
 (segment (start 69.5983 57.8542) (end 69.5983 59.3612) (width 1) (layer "B.Cu") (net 32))
 (segment (start 69.9183 56.0325) (end 69.9183 57.5342) (width 1) (layer "B.Cu") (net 32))
 (segment (start 77.5383 57.5342) (end 77.213 57.8595) (width 1) (layer "B.Cu") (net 29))
 (segment (start 77.213 57.8595) (end 77.0983 57.8595) (width 1) (layer "B.Cu") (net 29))
 (segment (start 77.5383 56.0325) (end 77.5383 57.5342) (width 1) (layer "B.Cu") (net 29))
 (segment (start 77.0983 59.3612) (end 77.0983 57.8595) (width 1) (layer "B.Cu") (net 29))
 (segment (start 54.6783 71.2725) (end 54.6783 72.7742) (width 1) (layer "B.Cu") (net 3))
 (segment (start 54.5983 72.8542) (end 54.5983 74.6012) (width 1) (layer "B.Cu") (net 3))
 (segment (start 54.6783 72.7742) (end 54.5983 72.8542) (width 1) (layer "B.Cu") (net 3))
 (segment (start 49.5983 56.0325) (end 49.5983 59.3612) (width 1) (layer "B.Cu") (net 40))
 (segment (start 52.1383 56.0325) (end 52.1383 57.5342) (width 1) (layer "B.Cu") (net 39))
 (segment (start 52.0983 57.5742) (end 52.0983 59.3612) (width 1) (layer "B.Cu") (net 39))
 (segment (start 52.1383 57.5342) (end 52.0983 57.5742) (width 1) (layer "B.Cu") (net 39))
 (segment (start 79.753 73.0995) (end 79.5983 73.0995) (width 1) (layer "B.Cu") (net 13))
 (segment (start 80.0783 72.7742) (end 79.753 73.0995) (width 1) (layer "B.Cu") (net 13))
 (segment (start 79.5983 74.6012) (end 79.5983 73.0995) (width 1) (layer "B.Cu") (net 13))
 (segment (start 80.0783 71.2725) (end 80.0783 72.7742) (width 1) (layer "B.Cu") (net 13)))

